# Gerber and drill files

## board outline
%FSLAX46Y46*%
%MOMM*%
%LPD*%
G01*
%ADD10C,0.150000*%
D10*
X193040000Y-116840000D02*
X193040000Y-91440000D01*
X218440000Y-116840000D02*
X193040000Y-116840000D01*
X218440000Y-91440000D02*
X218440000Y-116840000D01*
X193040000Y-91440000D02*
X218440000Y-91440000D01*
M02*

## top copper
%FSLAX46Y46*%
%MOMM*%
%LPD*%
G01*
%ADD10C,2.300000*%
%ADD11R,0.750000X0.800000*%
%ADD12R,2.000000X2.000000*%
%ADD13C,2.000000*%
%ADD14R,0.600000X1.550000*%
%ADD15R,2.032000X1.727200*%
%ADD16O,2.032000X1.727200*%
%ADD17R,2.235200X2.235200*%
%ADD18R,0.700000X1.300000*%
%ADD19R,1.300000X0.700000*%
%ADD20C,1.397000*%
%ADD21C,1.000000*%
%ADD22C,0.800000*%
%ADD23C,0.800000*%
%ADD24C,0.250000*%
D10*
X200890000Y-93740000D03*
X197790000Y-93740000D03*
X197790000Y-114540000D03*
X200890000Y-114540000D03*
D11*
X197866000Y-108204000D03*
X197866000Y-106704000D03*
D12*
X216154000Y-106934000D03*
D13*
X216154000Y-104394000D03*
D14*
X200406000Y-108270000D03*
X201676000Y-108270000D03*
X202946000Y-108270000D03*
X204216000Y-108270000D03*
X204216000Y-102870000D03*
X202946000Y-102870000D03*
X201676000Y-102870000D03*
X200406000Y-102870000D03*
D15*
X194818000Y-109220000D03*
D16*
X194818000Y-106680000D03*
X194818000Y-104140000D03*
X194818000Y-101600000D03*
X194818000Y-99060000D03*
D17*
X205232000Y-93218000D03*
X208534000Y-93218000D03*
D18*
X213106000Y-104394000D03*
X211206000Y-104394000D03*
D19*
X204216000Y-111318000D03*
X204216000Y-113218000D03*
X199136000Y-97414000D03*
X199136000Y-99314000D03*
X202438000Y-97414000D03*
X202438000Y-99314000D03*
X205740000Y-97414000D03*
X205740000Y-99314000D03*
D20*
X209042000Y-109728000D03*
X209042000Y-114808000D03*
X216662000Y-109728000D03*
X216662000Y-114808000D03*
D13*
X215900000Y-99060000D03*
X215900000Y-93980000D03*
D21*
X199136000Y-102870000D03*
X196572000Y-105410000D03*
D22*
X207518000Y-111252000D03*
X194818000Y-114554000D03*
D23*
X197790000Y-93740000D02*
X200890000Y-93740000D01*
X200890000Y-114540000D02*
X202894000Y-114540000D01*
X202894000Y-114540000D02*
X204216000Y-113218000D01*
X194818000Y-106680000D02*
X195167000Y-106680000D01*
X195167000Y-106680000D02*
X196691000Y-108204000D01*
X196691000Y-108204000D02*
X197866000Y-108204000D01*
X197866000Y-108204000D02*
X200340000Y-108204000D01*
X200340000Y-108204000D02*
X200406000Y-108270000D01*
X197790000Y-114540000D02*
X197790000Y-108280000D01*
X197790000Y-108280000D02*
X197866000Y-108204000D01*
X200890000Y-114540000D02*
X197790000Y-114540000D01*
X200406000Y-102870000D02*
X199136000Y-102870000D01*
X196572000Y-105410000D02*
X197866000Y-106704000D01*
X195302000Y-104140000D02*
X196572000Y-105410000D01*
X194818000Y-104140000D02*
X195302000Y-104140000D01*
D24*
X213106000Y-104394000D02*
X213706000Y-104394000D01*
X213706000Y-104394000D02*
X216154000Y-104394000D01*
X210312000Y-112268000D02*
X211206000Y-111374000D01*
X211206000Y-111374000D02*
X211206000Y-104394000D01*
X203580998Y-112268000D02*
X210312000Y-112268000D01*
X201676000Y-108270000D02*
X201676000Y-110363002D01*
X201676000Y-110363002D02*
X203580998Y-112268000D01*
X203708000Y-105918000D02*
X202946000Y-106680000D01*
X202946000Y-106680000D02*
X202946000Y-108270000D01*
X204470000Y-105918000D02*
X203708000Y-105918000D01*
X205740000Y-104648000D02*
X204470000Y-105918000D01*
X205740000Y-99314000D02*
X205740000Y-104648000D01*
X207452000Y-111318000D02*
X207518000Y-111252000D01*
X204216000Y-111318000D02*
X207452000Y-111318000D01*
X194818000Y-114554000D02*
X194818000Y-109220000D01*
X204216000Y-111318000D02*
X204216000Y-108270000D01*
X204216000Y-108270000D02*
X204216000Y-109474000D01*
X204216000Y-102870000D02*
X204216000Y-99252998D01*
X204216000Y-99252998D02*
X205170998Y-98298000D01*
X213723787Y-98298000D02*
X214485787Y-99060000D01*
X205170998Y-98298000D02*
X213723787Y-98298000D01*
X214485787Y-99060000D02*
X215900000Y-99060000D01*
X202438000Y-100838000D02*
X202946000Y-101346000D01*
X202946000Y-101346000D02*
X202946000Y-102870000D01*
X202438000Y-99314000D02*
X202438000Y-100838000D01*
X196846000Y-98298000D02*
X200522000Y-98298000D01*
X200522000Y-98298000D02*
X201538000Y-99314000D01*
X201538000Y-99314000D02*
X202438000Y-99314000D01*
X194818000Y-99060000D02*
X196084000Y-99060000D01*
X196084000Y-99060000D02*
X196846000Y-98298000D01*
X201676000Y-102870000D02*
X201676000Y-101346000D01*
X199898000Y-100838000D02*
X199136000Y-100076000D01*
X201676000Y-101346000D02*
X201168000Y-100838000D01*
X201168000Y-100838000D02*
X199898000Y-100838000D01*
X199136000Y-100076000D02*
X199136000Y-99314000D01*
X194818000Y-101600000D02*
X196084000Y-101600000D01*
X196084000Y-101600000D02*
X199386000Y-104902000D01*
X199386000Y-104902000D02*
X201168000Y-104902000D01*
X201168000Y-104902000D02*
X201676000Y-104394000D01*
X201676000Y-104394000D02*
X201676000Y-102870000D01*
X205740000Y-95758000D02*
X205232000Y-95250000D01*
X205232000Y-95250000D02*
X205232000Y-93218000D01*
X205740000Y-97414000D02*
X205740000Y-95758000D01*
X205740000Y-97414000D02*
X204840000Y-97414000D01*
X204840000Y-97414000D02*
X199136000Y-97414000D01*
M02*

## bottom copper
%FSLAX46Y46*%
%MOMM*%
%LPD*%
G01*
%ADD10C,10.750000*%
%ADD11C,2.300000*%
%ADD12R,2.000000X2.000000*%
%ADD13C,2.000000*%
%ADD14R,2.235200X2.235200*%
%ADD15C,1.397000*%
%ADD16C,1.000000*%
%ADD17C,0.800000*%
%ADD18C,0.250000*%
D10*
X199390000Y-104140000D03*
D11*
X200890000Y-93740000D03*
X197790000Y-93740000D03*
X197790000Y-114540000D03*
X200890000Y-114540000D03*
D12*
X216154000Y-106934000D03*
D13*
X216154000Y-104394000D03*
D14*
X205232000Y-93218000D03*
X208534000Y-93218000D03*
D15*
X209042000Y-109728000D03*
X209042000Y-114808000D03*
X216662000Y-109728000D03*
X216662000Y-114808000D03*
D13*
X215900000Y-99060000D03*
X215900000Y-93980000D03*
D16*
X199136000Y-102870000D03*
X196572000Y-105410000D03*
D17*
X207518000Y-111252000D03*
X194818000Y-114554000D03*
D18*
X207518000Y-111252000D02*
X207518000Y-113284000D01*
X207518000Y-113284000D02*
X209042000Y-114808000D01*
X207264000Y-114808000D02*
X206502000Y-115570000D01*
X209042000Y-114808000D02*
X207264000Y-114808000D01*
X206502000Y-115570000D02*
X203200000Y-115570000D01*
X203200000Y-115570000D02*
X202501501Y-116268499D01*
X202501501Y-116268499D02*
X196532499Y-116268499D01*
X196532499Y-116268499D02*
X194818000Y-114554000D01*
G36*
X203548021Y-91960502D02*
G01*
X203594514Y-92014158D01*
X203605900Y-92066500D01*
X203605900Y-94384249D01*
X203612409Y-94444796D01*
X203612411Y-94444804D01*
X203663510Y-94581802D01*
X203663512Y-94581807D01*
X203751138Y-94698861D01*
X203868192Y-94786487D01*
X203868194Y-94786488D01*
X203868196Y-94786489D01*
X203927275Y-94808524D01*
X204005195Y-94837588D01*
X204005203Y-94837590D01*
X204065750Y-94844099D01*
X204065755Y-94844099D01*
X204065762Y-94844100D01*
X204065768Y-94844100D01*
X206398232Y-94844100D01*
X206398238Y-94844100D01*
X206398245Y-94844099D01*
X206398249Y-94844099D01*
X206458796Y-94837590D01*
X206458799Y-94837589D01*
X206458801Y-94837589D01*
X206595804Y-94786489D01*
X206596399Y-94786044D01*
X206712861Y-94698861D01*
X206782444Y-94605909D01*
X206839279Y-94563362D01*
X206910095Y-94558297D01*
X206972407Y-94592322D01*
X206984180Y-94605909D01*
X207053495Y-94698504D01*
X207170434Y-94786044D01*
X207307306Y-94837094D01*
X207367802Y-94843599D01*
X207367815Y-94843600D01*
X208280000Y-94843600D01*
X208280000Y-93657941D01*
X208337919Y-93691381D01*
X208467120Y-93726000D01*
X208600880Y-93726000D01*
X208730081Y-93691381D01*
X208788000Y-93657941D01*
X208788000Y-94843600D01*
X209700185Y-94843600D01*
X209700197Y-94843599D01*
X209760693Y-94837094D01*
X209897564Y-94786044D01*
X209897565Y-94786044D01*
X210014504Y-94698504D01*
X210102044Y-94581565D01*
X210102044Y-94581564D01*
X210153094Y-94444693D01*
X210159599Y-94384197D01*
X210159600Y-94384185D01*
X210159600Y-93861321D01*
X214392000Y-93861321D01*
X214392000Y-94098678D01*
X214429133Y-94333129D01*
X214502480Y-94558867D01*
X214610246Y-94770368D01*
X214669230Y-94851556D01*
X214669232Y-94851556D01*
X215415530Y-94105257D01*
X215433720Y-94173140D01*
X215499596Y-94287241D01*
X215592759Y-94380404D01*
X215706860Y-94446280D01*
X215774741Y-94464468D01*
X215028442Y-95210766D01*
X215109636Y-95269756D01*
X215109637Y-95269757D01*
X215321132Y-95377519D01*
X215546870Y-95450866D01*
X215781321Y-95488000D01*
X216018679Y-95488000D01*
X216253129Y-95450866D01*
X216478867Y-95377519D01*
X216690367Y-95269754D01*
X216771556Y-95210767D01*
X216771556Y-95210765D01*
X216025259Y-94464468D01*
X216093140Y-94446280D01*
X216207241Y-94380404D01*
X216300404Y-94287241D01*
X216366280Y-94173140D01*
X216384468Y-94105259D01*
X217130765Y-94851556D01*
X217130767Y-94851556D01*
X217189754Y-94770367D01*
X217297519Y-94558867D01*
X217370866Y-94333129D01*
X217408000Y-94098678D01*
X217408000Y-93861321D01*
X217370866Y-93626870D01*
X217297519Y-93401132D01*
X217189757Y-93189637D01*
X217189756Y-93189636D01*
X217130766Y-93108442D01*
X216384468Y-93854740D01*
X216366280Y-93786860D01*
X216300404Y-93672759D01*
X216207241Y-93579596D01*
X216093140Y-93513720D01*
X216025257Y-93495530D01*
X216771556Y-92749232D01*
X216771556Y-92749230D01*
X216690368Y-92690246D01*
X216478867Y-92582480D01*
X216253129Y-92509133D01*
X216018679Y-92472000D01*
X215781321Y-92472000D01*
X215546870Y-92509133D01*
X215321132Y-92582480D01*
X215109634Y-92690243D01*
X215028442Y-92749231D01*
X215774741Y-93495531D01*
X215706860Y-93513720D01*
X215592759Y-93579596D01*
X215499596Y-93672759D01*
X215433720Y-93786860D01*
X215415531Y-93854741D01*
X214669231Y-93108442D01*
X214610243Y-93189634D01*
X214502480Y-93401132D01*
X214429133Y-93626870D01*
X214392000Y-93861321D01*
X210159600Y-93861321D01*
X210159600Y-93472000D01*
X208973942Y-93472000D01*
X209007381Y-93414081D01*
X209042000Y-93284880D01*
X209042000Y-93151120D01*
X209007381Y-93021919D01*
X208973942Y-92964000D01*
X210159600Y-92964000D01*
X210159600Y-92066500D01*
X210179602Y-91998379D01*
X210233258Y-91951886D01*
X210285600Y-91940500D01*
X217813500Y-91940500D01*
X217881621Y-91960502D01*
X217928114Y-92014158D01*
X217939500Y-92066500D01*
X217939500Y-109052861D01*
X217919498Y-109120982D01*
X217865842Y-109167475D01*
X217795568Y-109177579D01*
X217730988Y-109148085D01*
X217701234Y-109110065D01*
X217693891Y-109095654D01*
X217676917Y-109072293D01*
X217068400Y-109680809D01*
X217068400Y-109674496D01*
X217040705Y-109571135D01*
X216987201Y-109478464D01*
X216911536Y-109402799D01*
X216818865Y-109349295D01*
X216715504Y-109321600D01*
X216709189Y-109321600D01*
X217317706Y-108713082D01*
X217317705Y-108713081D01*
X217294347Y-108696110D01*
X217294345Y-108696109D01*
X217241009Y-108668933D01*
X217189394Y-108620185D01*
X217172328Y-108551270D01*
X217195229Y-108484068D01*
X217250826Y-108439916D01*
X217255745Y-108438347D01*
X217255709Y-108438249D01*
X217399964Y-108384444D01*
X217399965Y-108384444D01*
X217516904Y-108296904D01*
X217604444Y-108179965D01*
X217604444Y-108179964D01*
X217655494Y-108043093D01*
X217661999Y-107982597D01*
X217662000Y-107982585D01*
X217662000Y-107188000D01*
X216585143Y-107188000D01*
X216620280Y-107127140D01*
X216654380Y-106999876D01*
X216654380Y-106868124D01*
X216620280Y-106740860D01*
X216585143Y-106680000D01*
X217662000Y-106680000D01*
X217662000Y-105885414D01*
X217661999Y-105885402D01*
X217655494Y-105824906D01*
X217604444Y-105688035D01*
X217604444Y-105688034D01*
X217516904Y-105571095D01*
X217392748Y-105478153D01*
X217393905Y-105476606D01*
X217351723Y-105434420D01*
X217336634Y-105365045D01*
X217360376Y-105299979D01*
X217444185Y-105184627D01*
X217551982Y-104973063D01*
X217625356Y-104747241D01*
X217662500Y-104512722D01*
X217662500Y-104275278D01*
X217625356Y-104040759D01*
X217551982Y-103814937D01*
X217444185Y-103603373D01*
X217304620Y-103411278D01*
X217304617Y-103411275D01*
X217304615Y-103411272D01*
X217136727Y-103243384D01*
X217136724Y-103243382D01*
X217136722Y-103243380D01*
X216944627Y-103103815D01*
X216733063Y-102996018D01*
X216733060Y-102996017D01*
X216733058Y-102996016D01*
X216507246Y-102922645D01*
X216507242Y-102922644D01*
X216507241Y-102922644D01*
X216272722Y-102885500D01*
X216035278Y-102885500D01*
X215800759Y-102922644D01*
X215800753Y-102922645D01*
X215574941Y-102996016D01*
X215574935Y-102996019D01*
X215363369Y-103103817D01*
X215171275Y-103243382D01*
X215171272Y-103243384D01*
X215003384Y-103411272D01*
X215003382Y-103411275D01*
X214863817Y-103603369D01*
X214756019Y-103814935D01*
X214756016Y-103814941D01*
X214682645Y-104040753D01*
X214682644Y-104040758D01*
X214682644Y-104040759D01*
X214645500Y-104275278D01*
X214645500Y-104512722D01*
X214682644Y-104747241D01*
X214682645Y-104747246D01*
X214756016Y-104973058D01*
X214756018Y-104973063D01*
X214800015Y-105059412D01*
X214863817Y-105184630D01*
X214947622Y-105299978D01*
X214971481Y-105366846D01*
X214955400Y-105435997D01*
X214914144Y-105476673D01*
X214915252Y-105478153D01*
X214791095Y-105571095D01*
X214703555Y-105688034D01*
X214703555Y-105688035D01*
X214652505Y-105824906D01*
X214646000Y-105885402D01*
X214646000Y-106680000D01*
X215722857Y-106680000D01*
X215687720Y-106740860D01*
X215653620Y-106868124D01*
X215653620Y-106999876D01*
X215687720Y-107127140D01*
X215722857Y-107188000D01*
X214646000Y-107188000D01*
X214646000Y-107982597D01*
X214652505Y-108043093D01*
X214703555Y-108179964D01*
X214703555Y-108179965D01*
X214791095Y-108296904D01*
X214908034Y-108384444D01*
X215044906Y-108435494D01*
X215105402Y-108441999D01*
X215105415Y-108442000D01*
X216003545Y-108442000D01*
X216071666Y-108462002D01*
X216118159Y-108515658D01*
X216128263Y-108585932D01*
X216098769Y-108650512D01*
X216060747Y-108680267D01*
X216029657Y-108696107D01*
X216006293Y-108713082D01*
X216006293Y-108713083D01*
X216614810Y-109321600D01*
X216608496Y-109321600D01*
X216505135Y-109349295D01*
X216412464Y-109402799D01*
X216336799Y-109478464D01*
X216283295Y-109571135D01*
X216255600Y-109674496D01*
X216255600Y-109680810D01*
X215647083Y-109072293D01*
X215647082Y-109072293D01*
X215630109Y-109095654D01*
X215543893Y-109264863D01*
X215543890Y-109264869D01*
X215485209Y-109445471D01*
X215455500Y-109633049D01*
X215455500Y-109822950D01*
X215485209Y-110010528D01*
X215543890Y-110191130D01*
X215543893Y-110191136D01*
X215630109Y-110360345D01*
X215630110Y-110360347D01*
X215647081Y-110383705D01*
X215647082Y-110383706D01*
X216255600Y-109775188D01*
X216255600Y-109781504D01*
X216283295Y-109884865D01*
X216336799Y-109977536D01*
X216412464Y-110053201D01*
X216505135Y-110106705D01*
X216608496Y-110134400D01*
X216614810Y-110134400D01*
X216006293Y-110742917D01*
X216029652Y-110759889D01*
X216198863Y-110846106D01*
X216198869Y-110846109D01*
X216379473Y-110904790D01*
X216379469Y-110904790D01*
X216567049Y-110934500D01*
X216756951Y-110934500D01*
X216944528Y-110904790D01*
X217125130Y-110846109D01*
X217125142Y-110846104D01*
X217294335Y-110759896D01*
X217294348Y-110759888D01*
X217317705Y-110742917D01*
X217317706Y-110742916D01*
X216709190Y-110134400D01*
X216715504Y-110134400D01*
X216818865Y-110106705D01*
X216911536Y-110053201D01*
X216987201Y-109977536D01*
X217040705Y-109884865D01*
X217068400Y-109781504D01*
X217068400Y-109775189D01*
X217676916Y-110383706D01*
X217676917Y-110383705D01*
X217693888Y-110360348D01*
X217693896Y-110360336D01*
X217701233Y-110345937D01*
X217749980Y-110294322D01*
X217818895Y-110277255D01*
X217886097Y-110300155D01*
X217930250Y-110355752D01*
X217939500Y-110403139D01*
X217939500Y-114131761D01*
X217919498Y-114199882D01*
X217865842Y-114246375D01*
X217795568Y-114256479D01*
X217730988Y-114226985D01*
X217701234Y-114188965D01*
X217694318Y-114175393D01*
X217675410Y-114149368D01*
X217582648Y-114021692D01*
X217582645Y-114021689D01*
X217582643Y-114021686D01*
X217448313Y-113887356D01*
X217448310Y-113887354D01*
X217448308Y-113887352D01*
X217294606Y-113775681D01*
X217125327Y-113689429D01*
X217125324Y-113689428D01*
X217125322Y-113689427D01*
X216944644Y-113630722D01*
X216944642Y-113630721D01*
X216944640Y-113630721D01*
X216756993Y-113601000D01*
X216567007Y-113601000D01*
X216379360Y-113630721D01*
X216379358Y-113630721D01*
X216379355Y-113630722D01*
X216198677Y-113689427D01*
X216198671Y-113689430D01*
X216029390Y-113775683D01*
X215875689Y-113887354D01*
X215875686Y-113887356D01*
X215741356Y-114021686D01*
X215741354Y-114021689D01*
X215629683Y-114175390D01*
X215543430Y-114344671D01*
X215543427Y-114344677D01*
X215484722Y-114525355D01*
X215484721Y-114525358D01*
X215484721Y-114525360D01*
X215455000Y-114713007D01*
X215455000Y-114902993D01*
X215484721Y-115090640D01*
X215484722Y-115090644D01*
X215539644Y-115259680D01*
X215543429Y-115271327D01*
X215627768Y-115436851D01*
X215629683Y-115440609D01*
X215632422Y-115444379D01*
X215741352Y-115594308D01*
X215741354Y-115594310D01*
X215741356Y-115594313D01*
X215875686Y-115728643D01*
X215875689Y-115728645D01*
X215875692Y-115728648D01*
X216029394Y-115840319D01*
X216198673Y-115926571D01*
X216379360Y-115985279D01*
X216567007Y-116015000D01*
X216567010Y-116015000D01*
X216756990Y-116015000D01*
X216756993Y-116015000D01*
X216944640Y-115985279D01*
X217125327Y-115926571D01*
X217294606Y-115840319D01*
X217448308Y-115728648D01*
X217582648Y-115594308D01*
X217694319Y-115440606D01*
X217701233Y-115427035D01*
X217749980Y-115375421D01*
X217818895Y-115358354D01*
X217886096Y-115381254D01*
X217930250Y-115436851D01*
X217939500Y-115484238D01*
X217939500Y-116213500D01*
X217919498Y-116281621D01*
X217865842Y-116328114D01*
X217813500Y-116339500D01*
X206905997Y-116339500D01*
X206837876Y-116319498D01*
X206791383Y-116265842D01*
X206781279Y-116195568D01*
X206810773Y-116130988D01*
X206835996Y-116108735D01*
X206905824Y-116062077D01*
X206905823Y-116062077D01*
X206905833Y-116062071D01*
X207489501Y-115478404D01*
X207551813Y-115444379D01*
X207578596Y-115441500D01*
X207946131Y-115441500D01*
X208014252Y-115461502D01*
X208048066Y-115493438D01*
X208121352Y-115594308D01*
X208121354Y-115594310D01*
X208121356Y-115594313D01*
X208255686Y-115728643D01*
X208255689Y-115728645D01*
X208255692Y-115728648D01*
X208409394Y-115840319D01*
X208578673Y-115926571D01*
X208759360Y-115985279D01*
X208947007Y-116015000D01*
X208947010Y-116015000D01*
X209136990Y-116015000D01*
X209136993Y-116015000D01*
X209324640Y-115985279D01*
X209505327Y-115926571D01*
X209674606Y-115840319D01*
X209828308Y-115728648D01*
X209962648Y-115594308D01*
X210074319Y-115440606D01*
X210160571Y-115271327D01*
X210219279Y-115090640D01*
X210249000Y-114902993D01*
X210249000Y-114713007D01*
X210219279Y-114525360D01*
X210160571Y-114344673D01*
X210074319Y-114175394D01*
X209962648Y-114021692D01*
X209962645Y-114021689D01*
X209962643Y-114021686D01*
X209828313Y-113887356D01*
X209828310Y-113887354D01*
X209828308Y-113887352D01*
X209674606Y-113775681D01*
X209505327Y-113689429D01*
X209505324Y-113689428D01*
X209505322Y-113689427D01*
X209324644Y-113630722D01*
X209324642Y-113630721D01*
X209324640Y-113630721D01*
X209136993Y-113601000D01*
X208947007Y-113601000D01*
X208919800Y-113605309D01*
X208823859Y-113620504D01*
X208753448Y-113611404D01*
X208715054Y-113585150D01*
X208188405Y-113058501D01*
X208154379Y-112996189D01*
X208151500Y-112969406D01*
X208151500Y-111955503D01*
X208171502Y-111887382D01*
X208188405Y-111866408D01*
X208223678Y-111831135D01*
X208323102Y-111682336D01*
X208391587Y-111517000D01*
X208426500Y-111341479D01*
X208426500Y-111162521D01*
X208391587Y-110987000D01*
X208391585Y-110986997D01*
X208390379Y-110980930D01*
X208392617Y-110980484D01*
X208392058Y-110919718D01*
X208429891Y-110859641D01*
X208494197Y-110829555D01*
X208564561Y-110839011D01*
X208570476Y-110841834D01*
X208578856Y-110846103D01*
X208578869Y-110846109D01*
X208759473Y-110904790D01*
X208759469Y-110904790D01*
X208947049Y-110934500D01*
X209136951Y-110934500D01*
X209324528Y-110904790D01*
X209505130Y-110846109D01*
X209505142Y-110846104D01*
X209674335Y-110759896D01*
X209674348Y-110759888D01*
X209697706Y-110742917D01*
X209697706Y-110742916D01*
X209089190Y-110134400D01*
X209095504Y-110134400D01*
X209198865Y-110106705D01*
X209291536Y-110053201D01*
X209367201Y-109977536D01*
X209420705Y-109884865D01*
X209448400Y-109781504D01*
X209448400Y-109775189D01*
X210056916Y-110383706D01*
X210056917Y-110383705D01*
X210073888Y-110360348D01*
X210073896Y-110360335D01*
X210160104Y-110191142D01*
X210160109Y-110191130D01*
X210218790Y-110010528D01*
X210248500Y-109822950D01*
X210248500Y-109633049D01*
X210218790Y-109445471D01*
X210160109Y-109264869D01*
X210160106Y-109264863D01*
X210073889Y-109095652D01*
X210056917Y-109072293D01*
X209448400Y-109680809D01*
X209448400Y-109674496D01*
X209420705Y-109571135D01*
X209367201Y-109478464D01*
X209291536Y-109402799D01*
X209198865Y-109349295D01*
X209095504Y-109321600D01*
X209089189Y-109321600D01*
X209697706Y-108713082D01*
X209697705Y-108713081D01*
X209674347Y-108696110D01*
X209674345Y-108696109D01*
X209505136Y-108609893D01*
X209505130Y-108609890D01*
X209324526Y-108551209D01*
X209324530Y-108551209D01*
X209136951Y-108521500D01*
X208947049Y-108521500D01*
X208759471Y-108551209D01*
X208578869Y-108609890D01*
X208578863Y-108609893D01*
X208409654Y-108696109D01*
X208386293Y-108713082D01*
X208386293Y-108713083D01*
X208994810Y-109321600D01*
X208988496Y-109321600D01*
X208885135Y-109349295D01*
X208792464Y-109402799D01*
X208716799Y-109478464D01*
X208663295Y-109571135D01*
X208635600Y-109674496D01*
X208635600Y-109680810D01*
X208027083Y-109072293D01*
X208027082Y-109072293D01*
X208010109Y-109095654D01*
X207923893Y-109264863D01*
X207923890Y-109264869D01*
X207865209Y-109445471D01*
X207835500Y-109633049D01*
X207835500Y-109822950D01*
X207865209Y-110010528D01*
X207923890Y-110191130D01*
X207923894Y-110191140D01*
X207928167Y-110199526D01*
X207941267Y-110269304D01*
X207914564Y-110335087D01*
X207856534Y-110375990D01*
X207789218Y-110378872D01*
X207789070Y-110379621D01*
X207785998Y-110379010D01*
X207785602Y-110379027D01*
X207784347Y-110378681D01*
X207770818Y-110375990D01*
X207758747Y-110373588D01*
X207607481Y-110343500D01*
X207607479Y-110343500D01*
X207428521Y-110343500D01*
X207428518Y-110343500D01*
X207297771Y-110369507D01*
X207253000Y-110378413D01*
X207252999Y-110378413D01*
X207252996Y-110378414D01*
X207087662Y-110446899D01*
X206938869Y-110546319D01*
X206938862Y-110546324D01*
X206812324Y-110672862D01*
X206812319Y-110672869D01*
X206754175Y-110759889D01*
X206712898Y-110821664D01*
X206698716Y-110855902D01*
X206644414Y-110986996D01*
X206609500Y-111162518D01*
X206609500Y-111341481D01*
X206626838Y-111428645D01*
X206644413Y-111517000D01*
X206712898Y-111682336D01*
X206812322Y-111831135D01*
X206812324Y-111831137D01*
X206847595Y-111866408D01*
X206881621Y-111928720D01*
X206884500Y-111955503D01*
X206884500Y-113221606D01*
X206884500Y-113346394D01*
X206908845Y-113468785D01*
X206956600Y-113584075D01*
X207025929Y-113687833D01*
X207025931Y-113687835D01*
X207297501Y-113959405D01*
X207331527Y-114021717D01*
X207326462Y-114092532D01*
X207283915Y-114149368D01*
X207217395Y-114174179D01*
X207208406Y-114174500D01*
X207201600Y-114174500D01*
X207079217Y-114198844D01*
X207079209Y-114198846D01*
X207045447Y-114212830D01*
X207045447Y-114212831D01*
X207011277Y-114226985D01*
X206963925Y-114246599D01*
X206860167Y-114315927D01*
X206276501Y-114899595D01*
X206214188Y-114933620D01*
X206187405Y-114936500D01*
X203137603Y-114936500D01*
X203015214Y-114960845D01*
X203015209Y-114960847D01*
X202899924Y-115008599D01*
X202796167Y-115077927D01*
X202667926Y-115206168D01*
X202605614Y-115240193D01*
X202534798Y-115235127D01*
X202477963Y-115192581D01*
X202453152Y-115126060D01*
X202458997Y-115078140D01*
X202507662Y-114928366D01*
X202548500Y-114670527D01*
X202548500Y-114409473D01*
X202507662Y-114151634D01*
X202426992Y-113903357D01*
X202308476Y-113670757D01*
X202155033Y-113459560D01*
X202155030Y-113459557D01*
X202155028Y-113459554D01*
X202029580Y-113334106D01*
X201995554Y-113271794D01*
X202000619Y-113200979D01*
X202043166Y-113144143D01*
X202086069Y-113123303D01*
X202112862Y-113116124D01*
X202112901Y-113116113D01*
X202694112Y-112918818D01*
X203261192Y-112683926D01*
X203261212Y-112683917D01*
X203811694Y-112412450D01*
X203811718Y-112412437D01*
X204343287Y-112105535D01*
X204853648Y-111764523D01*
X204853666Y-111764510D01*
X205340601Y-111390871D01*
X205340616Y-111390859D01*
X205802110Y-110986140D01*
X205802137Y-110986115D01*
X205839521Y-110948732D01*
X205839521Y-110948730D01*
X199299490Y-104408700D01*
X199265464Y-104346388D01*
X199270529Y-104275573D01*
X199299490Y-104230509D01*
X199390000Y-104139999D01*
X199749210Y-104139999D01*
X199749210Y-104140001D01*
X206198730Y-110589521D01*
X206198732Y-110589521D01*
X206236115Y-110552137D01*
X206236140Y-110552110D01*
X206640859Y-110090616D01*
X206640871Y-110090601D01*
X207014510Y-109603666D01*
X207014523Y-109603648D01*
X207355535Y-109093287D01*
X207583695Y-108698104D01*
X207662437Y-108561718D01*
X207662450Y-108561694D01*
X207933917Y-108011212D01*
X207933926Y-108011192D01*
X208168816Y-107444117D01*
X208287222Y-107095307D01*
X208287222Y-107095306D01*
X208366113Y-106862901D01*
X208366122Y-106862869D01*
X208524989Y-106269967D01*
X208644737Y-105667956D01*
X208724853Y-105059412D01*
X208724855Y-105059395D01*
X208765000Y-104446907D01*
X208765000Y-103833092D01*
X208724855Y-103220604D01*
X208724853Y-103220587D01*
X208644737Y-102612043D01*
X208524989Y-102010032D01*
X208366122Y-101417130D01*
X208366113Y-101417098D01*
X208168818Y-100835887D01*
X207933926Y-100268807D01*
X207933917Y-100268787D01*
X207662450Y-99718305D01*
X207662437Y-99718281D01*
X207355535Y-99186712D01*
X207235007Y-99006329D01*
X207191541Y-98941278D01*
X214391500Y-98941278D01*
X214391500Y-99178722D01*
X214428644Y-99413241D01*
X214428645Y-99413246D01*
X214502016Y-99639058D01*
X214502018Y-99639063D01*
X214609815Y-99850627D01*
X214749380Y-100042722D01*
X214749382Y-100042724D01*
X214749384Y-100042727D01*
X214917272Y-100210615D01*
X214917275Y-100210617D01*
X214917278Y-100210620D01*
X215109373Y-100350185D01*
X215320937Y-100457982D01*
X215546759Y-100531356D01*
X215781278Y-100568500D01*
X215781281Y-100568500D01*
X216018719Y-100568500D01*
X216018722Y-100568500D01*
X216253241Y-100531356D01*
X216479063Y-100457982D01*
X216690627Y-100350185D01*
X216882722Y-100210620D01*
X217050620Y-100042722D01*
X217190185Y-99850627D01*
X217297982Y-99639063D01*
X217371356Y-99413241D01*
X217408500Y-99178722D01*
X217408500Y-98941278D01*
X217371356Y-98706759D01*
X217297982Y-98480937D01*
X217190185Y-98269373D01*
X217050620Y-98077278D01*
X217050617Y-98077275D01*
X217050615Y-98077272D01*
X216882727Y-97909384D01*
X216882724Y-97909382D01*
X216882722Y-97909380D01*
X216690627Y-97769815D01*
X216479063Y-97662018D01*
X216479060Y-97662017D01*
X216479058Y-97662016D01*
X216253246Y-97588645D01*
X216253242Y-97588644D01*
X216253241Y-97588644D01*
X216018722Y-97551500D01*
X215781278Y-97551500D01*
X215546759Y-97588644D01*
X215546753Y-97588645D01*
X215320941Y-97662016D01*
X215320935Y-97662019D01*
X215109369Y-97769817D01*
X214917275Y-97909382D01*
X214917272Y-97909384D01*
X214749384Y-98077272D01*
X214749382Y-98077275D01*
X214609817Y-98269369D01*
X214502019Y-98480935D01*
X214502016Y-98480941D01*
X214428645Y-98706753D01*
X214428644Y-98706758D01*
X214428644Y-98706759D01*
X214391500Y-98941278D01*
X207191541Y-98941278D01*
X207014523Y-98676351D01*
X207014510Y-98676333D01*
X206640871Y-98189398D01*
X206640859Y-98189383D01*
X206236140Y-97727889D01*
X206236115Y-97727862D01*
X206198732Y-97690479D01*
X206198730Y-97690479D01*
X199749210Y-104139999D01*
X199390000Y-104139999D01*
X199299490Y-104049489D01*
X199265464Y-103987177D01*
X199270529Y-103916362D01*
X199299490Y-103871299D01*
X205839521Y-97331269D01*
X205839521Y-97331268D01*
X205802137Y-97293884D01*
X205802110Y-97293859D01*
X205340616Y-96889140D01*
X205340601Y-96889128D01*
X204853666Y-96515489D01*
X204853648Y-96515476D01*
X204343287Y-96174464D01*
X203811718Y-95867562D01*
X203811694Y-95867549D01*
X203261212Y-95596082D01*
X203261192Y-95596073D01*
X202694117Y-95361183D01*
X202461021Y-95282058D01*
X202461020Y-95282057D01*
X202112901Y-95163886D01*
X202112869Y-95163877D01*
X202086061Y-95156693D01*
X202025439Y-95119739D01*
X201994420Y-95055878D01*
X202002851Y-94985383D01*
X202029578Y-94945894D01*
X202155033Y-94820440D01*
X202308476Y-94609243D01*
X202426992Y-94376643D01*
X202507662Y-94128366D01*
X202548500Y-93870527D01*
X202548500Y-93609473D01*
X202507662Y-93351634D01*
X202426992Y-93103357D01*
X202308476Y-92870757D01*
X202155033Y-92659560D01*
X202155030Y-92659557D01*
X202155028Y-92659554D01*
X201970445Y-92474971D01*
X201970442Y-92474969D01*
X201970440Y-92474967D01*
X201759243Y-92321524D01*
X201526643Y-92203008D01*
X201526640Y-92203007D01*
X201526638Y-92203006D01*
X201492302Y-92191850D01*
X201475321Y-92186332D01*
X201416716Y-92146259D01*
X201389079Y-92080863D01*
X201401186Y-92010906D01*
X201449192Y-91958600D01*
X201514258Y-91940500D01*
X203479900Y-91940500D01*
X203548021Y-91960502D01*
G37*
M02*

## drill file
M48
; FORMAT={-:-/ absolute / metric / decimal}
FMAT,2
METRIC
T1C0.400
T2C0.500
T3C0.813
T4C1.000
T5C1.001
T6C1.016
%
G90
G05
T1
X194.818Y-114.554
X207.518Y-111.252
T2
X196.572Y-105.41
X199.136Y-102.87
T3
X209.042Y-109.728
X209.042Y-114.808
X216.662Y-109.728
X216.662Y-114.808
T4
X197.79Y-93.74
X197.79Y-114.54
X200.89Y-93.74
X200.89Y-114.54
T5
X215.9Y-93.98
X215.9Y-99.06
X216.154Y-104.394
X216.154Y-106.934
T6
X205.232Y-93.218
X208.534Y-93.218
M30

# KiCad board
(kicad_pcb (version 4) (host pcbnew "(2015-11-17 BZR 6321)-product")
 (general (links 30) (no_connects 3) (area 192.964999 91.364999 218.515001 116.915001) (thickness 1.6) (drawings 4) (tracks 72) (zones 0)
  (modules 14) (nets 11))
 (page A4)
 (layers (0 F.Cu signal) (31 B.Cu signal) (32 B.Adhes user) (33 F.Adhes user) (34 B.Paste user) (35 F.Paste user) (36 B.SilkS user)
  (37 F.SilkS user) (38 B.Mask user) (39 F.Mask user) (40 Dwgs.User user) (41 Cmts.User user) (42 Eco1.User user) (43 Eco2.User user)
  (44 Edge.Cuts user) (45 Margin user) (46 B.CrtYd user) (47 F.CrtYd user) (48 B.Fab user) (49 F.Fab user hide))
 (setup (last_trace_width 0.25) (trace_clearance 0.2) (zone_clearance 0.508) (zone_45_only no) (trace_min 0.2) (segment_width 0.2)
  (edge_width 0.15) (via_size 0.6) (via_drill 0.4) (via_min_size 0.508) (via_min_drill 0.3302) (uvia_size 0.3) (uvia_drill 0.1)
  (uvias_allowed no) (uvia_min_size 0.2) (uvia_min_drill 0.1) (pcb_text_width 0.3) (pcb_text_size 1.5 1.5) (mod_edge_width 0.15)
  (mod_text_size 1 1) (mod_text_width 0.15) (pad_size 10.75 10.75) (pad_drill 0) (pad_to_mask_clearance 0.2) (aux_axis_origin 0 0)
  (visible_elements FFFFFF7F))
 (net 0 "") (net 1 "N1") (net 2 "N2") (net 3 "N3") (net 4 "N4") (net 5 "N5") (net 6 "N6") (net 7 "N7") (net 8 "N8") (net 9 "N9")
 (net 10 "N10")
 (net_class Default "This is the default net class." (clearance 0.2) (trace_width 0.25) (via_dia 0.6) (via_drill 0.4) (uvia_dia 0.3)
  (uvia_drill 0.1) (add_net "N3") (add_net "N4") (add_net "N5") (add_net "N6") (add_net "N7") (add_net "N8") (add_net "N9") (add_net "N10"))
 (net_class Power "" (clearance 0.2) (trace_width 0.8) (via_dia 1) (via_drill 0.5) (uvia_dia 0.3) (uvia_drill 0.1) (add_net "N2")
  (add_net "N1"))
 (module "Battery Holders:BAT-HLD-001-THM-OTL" (layer B.Cu) (at 199.39 104.14 90)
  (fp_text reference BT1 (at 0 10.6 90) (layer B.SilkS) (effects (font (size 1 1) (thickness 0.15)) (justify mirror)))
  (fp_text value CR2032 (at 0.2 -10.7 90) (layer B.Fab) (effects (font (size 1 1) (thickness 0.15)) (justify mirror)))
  (pad 2 smd circle (at 0 0 90) (size 10.75 10.75) (layers B.Cu B.Mask) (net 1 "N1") (solder_mask_margin 4) (clearance 2.5) (zone_connect 1)
   (thermal_gap 4))
  (pad 1 thru_hole circle (at 10.4 1.5 90) (size 2.3 2.3) (drill 1) (layers *.Cu *.Mask B.SilkS) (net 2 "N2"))
  (pad 1 thru_hole circle (at 10.4 -1.6 90) (size 2.3 2.3) (drill 1) (layers *.Cu *.Mask B.SilkS) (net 2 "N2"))
  (pad 1 thru_hole circle (at -10.4 -1.6 90) (size 2.3 2.3) (drill 1) (layers *.Cu *.Mask B.SilkS) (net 2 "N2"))
  (pad 1 thru_hole circle (at -10.4 1.5 90) (size 2.3 2.3) (drill 1) (layers *.Cu *.Mask B.SilkS) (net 2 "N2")))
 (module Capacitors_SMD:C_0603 (layer F.Cu) (at 197.866 107.454 90)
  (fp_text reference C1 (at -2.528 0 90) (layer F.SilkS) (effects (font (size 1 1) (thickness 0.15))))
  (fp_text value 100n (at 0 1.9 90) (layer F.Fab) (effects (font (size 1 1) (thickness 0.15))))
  (pad 1 smd rect (at -0.75 0 90) (size 0.8 0.75) (layers F.Cu F.Paste F.Mask) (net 2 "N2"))
  (pad 2 smd rect (at 0.75 0 90) (size 0.8 0.75) (layers F.Cu F.Paste F.Mask) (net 1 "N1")))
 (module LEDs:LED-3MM (layer B.Cu) (at 216.154 106.934 90)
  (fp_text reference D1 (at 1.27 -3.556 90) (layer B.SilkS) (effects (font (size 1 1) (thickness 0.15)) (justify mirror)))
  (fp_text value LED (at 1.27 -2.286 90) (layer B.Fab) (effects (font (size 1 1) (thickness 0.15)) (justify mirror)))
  (pad 1 thru_hole rect (at 0 0) (size 2 2) (drill 1.00076) (layers *.Cu *.Mask B.SilkS) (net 1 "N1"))
  (pad 2 thru_hole circle (at 2.54 0 90) (size 2 2) (drill 1.00076) (layers *.Cu *.Mask B.SilkS) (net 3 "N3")))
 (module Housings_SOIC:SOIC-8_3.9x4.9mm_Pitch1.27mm (layer F.Cu) (at 202.311 105.57 90)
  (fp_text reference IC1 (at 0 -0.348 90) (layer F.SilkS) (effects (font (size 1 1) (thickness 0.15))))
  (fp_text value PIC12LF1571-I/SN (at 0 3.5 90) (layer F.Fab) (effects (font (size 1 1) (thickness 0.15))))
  (pad 1 smd rect (at -2.7 -1.905 90) (size 1.55 0.6) (layers F.Cu F.Paste F.Mask) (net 2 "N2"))
  (pad 2 smd rect (at -2.7 -0.635 90) (size 1.55 0.6) (layers F.Cu F.Paste F.Mask) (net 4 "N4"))
  (pad 3 smd rect (at -2.7 0.635 90) (size 1.55 0.6) (layers F.Cu F.Paste F.Mask) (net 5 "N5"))
  (pad 4 smd rect (at -2.7 1.905 90) (size 1.55 0.6) (layers F.Cu F.Paste F.Mask) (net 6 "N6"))
  (pad 5 smd rect (at 2.7 1.905 90) (size 1.55 0.6) (layers F.Cu F.Paste F.Mask) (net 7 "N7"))
  (pad 6 smd rect (at 2.7 0.635 90) (size 1.55 0.6) (layers F.Cu F.Paste F.Mask) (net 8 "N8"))
  (pad 7 smd rect (at 2.7 -0.635 90) (size 1.55 0.6) (layers F.Cu F.Paste F.Mask) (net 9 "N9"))
  (pad 8 smd rect (at 2.7 -1.905 90) (size 1.55 0.6) (layers F.Cu F.Paste F.Mask) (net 1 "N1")))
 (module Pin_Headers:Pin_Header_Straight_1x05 (layer F.Cu) (at 194.818 109.22 180)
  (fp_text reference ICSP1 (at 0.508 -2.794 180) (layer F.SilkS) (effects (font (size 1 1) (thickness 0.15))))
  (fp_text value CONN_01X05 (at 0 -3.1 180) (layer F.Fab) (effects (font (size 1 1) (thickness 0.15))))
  (pad 1 smd rect (at 0 0 180) (size 2.032 1.7272) (layers F.Cu F.Paste F.Mask) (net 6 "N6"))
  (pad 2 smd oval (at 0 2.54 180) (size 2.032 1.7272) (layers F.Cu F.Paste F.Mask) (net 2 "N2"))
  (pad 3 smd oval (at 0 5.08 180) (size 2.032 1.7272) (layers F.Cu F.Paste F.Mask) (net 1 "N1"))
  (pad 4 smd oval (at 0 7.62 180) (size 2.032 1.7272) (layers F.Cu F.Paste F.Mask) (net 9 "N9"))
  (pad 5 smd oval (at 0 10.16 180) (size 2.032 1.7272) (layers F.Cu F.Paste F.Mask) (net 8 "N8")))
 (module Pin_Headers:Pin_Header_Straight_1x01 (layer F.Cu) (at 205.232 93.218)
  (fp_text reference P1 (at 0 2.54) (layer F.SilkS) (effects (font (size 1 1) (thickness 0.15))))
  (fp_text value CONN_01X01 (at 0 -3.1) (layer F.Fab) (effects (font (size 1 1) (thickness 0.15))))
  (pad 1 thru_hole rect (at 0 0) (size 2.2352 2.2352) (drill 1.016) (layers *.Cu *.Mask F.SilkS) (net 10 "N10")))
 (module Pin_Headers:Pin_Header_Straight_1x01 (layer F.Cu) (at 208.534 93.218)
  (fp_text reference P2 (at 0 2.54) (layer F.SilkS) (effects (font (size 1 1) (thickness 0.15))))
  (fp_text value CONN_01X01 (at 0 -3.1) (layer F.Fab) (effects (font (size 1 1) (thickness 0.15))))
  (pad 1 thru_hole rect (at 0 0) (size 2.2352 2.2352) (drill 1.016) (layers *.Cu *.Mask F.SilkS) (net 1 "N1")))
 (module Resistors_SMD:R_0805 (layer F.Cu) (at 212.156 104.394 180)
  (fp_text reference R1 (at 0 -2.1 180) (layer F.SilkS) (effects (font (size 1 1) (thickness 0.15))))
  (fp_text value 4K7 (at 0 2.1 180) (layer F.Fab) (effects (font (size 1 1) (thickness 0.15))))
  (pad 1 smd rect (at -0.95 0 180) (size 0.7 1.3) (layers F.Cu F.Paste F.Mask) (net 3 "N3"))
  (pad 2 smd rect (at 0.95 0 180) (size 0.7 1.3) (layers F.Cu F.Paste F.Mask) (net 4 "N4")))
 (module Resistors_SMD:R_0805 (layer F.Cu) (at 204.216 112.268 270)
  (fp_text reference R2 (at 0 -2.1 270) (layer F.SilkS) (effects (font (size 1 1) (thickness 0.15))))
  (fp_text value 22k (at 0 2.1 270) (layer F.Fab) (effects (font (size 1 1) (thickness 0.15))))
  (pad 1 smd rect (at -0.95 0 270) (size 0.7 1.3) (layers F.Cu F.Paste F.Mask) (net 6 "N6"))
  (pad 2 smd rect (at 0.95 0 270) (size 0.7 1.3) (layers F.Cu F.Paste F.Mask) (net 2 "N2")))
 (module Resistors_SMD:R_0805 (layer F.Cu) (at 199.136 98.364 270)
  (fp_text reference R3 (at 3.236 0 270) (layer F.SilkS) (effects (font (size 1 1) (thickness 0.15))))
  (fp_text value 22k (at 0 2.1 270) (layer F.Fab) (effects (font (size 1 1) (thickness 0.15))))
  (pad 1 smd rect (at -0.95 0 270) (size 0.7 1.3) (layers F.Cu F.Paste F.Mask) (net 10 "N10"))
  (pad 2 smd rect (at 0.95 0 270) (size 0.7 1.3) (layers F.Cu F.Paste F.Mask) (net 9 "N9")))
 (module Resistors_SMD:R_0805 (layer F.Cu) (at 202.438 98.364 270)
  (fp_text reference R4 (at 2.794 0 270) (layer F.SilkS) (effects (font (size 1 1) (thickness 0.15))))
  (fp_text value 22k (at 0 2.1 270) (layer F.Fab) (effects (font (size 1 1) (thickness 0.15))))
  (pad 1 smd rect (at -0.95 0 270) (size 0.7 1.3) (layers F.Cu F.Paste F.Mask) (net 10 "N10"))
  (pad 2 smd rect (at 0.95 0 270) (size 0.7 1.3) (layers F.Cu F.Paste F.Mask) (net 8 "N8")))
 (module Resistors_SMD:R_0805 (layer F.Cu) (at 205.74 98.364 270)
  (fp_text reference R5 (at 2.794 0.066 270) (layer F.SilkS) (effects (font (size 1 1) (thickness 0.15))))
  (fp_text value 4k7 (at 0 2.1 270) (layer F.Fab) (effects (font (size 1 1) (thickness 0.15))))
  (pad 1 smd rect (at -0.95 0 270) (size 0.7 1.3) (layers F.Cu F.Paste F.Mask) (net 10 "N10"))
  (pad 2 smd rect (at 0.95 0 270) (size 0.7 1.3) (layers F.Cu F.Paste F.Mask) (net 5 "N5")))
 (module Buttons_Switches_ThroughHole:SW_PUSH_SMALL (layer B.Cu) (at 212.852 112.268 180)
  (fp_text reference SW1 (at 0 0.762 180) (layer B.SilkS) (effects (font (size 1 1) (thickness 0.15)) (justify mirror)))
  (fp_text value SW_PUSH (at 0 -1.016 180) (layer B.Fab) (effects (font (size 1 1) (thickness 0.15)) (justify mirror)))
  (pad 1 thru_hole circle (at 3.81 2.54 180) (size 1.397 1.397) (drill 0.8128) (layers *.Cu *.Mask B.SilkS) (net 1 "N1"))
  (pad 2 thru_hole circle (at 3.81 -2.54 180) (size 1.397 1.397) (drill 0.8128) (layers *.Cu *.Mask B.SilkS) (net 6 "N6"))
  (pad 1 thru_hole circle (at -3.81 2.54 180) (size 1.397 1.397) (drill 0.8128) (layers *.Cu *.Mask B.SilkS) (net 1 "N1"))
  (pad 2 thru_hole circle (at -3.81 -2.54 180) (size 1.397 1.397) (drill 0.8128) (layers *.Cu *.Mask B.SilkS) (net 6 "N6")))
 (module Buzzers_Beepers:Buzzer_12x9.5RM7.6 (layer B.Cu) (at 215.9 96.53016 90)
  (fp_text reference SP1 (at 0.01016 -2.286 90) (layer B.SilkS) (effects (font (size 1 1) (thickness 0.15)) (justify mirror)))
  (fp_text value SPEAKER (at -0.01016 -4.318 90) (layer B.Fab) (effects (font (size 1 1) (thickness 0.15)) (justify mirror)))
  (pad 1 thru_hole circle (at -2.52984 0 90) (size 2 2) (drill 1.00076) (layers *.Cu *.Mask B.SilkS) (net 7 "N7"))
  (pad 2 thru_hole circle (at 2.55016 0 90) (size 2 2) (drill 1.00076) (layers *.Cu *.Mask B.SilkS) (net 1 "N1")))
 (gr_line (start 193.04 116.84) (end 193.04 91.44) (layer Edge.Cuts) (width 0.15))
 (gr_line (start 218.44 116.84) (end 193.04 116.84) (layer Edge.Cuts) (width 0.15))
 (gr_line (start 218.44 91.44) (end 218.44 116.84) (layer Edge.Cuts) (width 0.15))
 (gr_line (start 193.04 91.44) (end 218.44 91.44) (layer Edge.Cuts) (width 0.15))
 (segment (start 197.79 93.74) (end 200.89 93.74) (width 0.8) (layer F.Cu) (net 2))
 (segment (start 200.89 114.54) (end 202.894 114.54) (width 0.8) (layer F.Cu) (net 2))
 (segment (start 202.894 114.54) (end 204.216 113.218) (width 0.8) (layer F.Cu) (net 2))
 (segment (start 194.818 106.68) (end 195.167 106.68) (width 0.8) (layer F.Cu) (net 2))
 (segment (start 195.167 106.68) (end 196.691 108.204) (width 0.8) (layer F.Cu) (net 2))
 (segment (start 196.691 108.204) (end 197.866 108.204) (width 0.8) (layer F.Cu) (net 2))
 (segment (start 197.866 108.204) (end 200.34 108.204) (width 0.8) (layer F.Cu) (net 2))
 (segment (start 200.34 108.204) (end 200.406 108.27) (width 0.8) (layer F.Cu) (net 2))
 (segment (start 197.79 114.54) (end 197.79 108.28) (width 0.8) (layer F.Cu) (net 2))
 (segment (start 197.79 108.28) (end 197.866 108.204) (width 0.8) (layer F.Cu) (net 2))
 (segment (start 200.89 114.54) (end 197.79 114.54) (width 0.8) (layer F.Cu) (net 2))
 (segment (start 200.406 102.87) (end 199.136 102.87) (width 0.8) (layer F.Cu) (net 1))
 (via (at 199.136 102.87) (size 1) (drill 0.5) (layers F.Cu B.Cu) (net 1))
 (segment (start 196.572 105.41) (end 197.866 106.704) (width 0.8) (layer F.Cu) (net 1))
 (segment (start 195.302 104.14) (end 196.572 105.41) (width 0.8) (layer F.Cu) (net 1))
 (via (at 196.572 105.41) (size 1) (drill 0.5) (layers F.Cu B.Cu) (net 1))
 (segment (start 194.818 104.14) (end 195.302 104.14) (width 0.8) (layer F.Cu) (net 1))
 (segment (start 213.106 104.394) (end 213.706 104.394) (width 0.25) (layer F.Cu) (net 3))
 (segment (start 213.706 104.394) (end 216.154 104.394) (width 0.25) (layer F.Cu) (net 3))
 (segment (start 210.312 112.268) (end 211.206 111.374) (width 0.25) (layer F.Cu) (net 4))
 (segment (start 211.206 111.374) (end 211.206 104.394) (width 0.25) (layer F.Cu) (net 4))
 (segment (start 203.580998 112.268) (end 210.312 112.268) (width 0.25) (layer F.Cu) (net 4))
 (segment (start 201.676 108.27) (end 201.676 110.363002) (width 0.25) (layer F.Cu) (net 4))
 (segment (start 201.676 110.363002) (end 203.580998 112.268) (width 0.25) (layer F.Cu) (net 4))
 (segment (start 203.708 105.918) (end 202.946 106.68) (width 0.25) (layer F.Cu) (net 5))
 (segment (start 202.946 106.68) (end 202.946 108.27) (width 0.25) (layer F.Cu) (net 5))
 (segment (start 204.47 105.918) (end 203.708 105.918) (width 0.25) (layer F.Cu) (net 5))
 (segment (start 205.74 104.648) (end 204.47 105.918) (width 0.25) (layer F.Cu) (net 5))
 (segment (start 205.74 99.314) (end 205.74 104.648) (width 0.25) (layer F.Cu) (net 5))
 (segment (start 207.518 111.252) (end 207.518 113.284) (width 0.25) (layer B.Cu) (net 6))
 (segment (start 207.518 113.284) (end 209.042 114.808) (width 0.25) (layer B.Cu) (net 6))
 (segment (start 207.264 114.808) (end 206.502 115.57) (width 0.25) (layer B.Cu) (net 6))
 (segment (start 209.042 114.808) (end 207.264 114.808) (width 0.25) (layer B.Cu) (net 6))
 (segment (start 206.502 115.57) (end 203.2 115.57) (width 0.25) (layer B.Cu) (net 6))
 (segment (start 203.2 115.57) (end 202.501501 116.268499) (width 0.25) (layer B.Cu) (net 6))
 (segment (start 202.501501 116.268499) (end 196.532499 116.268499) (width 0.25) (layer B.Cu) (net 6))
 (segment (start 196.532499 116.268499) (end 194.818 114.554) (width 0.25) (layer B.Cu) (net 6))
 (segment (start 207.452 111.318) (end 207.518 111.252) (width 0.25) (layer F.Cu) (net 6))
 (segment (start 204.216 111.318) (end 207.452 111.318) (width 0.25) (layer F.Cu) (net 6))
 (via (at 207.518 111.252) (size 0.8) (drill 0.4) (layers F.Cu B.Cu) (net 6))
 (segment (start 194.818 114.554) (end 194.818 109.22) (width 0.25) (layer F.Cu) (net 6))
 (via (at 194.818 114.554) (size 0.8) (drill 0.4) (layers F.Cu B.Cu) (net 6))
 (segment (start 204.216 111.318) (end 204.216 108.27) (width 0.25) (layer F.Cu) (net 6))
 (segment (start 204.216 108.27) (end 204.216 109.474) (width 0.25) (layer F.Cu) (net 6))
 (segment (start 204.216 102.87) (end 204.216 99.252998) (width 0.25) (layer F.Cu) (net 7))
 (segment (start 204.216 99.252998) (end 205.170998 98.298) (width 0.25) (layer F.Cu) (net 7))
 (segment (start 213.723787 98.298) (end 214.485787 99.06) (width 0.25) (layer F.Cu) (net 7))
 (segment (start 205.170998 98.298) (end 213.723787 98.298) (width 0.25) (layer F.Cu) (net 7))
 (segment (start 214.485787 99.06) (end 215.9 99.06) (width 0.25) (layer F.Cu) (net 7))
 (segment (start 202.438 100.838) (end 202.946 101.346) (width 0.25) (layer F.Cu) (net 8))
 (segment (start 202.946 101.346) (end 202.946 102.87) (width 0.25) (layer F.Cu) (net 8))
 (segment (start 202.438 99.314) (end 202.438 100.838) (width 0.25) (layer F.Cu) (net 8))
 (segment (start 196.846 98.298) (end 200.522 98.298) (width 0.25) (layer F.Cu) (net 8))
 (segment (start 200.522 98.298) (end 201.538 99.314) (width 0.25) (layer F.Cu) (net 8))
 (segment (start 201.538 99.314) (end 202.438 99.314) (width 0.25) (layer F.Cu) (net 8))
 (segment (start 194.818 99.06) (end 196.084 99.06) (width 0.25) (layer F.Cu) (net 8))
 (segment (start 196.084 99.06) (end 196.846 98.298) (width 0.25) (layer F.Cu) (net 8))
 (segment (start 201.676 102.87) (end 201.676 101.346) (width 0.25) (layer F.Cu) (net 9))
 (segment (start 199.898 100.838) (end 199.136 100.076) (width 0.25) (layer F.Cu) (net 9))
 (segment (start 201.676 101.346) (end 201.168 100.838) (width 0.25) (layer F.Cu) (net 9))
 (segment (start 201.168 100.838) (end 199.898 100.838) (width 0.25) (layer F.Cu) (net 9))
 (segment (start 199.136 100.076) (end 199.136 99.314) (width 0.25) (layer F.Cu) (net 9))
 (segment (start 194.818 101.6) (end 196.084 101.6) (width 0.25) (layer F.Cu) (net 9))
 (segment (start 196.084 101.6) (end 199.386 104.902) (width 0.25) (layer F.Cu) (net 9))
 (segment (start 199.386 104.902) (end 201.168 104.902) (width 0.25) (layer F.Cu) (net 9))
 (segment (start 201.168 104.902) (end 201.676 104.394) (width 0.25) (layer F.Cu) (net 9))
 (segment (start 201.676 104.394) (end 201.676 102.87) (width 0.25) (layer F.Cu) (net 9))
 (segment (start 205.74 95.758) (end 205.232 95.25) (width 0.25) (layer F.Cu) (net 10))
 (segment (start 205.232 95.25) (end 205.232 93.218) (width 0.25) (layer F.Cu) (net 10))
 (segment (start 205.74 97.414) (end 205.74 95.758) (width 0.25) (layer F.Cu) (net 10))
 (segment (start 205.74 97.414) (end 204.84 97.414) (width 0.25) (layer F.Cu) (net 10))
 (segment (start 204.84 97.414) (end 199.136 97.414) (width 0.25) (layer F.Cu) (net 10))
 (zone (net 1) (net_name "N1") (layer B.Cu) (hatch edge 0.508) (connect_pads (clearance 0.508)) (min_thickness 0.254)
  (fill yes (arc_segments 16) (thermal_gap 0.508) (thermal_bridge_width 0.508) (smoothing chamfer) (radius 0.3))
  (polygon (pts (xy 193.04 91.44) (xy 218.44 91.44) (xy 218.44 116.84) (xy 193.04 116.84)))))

